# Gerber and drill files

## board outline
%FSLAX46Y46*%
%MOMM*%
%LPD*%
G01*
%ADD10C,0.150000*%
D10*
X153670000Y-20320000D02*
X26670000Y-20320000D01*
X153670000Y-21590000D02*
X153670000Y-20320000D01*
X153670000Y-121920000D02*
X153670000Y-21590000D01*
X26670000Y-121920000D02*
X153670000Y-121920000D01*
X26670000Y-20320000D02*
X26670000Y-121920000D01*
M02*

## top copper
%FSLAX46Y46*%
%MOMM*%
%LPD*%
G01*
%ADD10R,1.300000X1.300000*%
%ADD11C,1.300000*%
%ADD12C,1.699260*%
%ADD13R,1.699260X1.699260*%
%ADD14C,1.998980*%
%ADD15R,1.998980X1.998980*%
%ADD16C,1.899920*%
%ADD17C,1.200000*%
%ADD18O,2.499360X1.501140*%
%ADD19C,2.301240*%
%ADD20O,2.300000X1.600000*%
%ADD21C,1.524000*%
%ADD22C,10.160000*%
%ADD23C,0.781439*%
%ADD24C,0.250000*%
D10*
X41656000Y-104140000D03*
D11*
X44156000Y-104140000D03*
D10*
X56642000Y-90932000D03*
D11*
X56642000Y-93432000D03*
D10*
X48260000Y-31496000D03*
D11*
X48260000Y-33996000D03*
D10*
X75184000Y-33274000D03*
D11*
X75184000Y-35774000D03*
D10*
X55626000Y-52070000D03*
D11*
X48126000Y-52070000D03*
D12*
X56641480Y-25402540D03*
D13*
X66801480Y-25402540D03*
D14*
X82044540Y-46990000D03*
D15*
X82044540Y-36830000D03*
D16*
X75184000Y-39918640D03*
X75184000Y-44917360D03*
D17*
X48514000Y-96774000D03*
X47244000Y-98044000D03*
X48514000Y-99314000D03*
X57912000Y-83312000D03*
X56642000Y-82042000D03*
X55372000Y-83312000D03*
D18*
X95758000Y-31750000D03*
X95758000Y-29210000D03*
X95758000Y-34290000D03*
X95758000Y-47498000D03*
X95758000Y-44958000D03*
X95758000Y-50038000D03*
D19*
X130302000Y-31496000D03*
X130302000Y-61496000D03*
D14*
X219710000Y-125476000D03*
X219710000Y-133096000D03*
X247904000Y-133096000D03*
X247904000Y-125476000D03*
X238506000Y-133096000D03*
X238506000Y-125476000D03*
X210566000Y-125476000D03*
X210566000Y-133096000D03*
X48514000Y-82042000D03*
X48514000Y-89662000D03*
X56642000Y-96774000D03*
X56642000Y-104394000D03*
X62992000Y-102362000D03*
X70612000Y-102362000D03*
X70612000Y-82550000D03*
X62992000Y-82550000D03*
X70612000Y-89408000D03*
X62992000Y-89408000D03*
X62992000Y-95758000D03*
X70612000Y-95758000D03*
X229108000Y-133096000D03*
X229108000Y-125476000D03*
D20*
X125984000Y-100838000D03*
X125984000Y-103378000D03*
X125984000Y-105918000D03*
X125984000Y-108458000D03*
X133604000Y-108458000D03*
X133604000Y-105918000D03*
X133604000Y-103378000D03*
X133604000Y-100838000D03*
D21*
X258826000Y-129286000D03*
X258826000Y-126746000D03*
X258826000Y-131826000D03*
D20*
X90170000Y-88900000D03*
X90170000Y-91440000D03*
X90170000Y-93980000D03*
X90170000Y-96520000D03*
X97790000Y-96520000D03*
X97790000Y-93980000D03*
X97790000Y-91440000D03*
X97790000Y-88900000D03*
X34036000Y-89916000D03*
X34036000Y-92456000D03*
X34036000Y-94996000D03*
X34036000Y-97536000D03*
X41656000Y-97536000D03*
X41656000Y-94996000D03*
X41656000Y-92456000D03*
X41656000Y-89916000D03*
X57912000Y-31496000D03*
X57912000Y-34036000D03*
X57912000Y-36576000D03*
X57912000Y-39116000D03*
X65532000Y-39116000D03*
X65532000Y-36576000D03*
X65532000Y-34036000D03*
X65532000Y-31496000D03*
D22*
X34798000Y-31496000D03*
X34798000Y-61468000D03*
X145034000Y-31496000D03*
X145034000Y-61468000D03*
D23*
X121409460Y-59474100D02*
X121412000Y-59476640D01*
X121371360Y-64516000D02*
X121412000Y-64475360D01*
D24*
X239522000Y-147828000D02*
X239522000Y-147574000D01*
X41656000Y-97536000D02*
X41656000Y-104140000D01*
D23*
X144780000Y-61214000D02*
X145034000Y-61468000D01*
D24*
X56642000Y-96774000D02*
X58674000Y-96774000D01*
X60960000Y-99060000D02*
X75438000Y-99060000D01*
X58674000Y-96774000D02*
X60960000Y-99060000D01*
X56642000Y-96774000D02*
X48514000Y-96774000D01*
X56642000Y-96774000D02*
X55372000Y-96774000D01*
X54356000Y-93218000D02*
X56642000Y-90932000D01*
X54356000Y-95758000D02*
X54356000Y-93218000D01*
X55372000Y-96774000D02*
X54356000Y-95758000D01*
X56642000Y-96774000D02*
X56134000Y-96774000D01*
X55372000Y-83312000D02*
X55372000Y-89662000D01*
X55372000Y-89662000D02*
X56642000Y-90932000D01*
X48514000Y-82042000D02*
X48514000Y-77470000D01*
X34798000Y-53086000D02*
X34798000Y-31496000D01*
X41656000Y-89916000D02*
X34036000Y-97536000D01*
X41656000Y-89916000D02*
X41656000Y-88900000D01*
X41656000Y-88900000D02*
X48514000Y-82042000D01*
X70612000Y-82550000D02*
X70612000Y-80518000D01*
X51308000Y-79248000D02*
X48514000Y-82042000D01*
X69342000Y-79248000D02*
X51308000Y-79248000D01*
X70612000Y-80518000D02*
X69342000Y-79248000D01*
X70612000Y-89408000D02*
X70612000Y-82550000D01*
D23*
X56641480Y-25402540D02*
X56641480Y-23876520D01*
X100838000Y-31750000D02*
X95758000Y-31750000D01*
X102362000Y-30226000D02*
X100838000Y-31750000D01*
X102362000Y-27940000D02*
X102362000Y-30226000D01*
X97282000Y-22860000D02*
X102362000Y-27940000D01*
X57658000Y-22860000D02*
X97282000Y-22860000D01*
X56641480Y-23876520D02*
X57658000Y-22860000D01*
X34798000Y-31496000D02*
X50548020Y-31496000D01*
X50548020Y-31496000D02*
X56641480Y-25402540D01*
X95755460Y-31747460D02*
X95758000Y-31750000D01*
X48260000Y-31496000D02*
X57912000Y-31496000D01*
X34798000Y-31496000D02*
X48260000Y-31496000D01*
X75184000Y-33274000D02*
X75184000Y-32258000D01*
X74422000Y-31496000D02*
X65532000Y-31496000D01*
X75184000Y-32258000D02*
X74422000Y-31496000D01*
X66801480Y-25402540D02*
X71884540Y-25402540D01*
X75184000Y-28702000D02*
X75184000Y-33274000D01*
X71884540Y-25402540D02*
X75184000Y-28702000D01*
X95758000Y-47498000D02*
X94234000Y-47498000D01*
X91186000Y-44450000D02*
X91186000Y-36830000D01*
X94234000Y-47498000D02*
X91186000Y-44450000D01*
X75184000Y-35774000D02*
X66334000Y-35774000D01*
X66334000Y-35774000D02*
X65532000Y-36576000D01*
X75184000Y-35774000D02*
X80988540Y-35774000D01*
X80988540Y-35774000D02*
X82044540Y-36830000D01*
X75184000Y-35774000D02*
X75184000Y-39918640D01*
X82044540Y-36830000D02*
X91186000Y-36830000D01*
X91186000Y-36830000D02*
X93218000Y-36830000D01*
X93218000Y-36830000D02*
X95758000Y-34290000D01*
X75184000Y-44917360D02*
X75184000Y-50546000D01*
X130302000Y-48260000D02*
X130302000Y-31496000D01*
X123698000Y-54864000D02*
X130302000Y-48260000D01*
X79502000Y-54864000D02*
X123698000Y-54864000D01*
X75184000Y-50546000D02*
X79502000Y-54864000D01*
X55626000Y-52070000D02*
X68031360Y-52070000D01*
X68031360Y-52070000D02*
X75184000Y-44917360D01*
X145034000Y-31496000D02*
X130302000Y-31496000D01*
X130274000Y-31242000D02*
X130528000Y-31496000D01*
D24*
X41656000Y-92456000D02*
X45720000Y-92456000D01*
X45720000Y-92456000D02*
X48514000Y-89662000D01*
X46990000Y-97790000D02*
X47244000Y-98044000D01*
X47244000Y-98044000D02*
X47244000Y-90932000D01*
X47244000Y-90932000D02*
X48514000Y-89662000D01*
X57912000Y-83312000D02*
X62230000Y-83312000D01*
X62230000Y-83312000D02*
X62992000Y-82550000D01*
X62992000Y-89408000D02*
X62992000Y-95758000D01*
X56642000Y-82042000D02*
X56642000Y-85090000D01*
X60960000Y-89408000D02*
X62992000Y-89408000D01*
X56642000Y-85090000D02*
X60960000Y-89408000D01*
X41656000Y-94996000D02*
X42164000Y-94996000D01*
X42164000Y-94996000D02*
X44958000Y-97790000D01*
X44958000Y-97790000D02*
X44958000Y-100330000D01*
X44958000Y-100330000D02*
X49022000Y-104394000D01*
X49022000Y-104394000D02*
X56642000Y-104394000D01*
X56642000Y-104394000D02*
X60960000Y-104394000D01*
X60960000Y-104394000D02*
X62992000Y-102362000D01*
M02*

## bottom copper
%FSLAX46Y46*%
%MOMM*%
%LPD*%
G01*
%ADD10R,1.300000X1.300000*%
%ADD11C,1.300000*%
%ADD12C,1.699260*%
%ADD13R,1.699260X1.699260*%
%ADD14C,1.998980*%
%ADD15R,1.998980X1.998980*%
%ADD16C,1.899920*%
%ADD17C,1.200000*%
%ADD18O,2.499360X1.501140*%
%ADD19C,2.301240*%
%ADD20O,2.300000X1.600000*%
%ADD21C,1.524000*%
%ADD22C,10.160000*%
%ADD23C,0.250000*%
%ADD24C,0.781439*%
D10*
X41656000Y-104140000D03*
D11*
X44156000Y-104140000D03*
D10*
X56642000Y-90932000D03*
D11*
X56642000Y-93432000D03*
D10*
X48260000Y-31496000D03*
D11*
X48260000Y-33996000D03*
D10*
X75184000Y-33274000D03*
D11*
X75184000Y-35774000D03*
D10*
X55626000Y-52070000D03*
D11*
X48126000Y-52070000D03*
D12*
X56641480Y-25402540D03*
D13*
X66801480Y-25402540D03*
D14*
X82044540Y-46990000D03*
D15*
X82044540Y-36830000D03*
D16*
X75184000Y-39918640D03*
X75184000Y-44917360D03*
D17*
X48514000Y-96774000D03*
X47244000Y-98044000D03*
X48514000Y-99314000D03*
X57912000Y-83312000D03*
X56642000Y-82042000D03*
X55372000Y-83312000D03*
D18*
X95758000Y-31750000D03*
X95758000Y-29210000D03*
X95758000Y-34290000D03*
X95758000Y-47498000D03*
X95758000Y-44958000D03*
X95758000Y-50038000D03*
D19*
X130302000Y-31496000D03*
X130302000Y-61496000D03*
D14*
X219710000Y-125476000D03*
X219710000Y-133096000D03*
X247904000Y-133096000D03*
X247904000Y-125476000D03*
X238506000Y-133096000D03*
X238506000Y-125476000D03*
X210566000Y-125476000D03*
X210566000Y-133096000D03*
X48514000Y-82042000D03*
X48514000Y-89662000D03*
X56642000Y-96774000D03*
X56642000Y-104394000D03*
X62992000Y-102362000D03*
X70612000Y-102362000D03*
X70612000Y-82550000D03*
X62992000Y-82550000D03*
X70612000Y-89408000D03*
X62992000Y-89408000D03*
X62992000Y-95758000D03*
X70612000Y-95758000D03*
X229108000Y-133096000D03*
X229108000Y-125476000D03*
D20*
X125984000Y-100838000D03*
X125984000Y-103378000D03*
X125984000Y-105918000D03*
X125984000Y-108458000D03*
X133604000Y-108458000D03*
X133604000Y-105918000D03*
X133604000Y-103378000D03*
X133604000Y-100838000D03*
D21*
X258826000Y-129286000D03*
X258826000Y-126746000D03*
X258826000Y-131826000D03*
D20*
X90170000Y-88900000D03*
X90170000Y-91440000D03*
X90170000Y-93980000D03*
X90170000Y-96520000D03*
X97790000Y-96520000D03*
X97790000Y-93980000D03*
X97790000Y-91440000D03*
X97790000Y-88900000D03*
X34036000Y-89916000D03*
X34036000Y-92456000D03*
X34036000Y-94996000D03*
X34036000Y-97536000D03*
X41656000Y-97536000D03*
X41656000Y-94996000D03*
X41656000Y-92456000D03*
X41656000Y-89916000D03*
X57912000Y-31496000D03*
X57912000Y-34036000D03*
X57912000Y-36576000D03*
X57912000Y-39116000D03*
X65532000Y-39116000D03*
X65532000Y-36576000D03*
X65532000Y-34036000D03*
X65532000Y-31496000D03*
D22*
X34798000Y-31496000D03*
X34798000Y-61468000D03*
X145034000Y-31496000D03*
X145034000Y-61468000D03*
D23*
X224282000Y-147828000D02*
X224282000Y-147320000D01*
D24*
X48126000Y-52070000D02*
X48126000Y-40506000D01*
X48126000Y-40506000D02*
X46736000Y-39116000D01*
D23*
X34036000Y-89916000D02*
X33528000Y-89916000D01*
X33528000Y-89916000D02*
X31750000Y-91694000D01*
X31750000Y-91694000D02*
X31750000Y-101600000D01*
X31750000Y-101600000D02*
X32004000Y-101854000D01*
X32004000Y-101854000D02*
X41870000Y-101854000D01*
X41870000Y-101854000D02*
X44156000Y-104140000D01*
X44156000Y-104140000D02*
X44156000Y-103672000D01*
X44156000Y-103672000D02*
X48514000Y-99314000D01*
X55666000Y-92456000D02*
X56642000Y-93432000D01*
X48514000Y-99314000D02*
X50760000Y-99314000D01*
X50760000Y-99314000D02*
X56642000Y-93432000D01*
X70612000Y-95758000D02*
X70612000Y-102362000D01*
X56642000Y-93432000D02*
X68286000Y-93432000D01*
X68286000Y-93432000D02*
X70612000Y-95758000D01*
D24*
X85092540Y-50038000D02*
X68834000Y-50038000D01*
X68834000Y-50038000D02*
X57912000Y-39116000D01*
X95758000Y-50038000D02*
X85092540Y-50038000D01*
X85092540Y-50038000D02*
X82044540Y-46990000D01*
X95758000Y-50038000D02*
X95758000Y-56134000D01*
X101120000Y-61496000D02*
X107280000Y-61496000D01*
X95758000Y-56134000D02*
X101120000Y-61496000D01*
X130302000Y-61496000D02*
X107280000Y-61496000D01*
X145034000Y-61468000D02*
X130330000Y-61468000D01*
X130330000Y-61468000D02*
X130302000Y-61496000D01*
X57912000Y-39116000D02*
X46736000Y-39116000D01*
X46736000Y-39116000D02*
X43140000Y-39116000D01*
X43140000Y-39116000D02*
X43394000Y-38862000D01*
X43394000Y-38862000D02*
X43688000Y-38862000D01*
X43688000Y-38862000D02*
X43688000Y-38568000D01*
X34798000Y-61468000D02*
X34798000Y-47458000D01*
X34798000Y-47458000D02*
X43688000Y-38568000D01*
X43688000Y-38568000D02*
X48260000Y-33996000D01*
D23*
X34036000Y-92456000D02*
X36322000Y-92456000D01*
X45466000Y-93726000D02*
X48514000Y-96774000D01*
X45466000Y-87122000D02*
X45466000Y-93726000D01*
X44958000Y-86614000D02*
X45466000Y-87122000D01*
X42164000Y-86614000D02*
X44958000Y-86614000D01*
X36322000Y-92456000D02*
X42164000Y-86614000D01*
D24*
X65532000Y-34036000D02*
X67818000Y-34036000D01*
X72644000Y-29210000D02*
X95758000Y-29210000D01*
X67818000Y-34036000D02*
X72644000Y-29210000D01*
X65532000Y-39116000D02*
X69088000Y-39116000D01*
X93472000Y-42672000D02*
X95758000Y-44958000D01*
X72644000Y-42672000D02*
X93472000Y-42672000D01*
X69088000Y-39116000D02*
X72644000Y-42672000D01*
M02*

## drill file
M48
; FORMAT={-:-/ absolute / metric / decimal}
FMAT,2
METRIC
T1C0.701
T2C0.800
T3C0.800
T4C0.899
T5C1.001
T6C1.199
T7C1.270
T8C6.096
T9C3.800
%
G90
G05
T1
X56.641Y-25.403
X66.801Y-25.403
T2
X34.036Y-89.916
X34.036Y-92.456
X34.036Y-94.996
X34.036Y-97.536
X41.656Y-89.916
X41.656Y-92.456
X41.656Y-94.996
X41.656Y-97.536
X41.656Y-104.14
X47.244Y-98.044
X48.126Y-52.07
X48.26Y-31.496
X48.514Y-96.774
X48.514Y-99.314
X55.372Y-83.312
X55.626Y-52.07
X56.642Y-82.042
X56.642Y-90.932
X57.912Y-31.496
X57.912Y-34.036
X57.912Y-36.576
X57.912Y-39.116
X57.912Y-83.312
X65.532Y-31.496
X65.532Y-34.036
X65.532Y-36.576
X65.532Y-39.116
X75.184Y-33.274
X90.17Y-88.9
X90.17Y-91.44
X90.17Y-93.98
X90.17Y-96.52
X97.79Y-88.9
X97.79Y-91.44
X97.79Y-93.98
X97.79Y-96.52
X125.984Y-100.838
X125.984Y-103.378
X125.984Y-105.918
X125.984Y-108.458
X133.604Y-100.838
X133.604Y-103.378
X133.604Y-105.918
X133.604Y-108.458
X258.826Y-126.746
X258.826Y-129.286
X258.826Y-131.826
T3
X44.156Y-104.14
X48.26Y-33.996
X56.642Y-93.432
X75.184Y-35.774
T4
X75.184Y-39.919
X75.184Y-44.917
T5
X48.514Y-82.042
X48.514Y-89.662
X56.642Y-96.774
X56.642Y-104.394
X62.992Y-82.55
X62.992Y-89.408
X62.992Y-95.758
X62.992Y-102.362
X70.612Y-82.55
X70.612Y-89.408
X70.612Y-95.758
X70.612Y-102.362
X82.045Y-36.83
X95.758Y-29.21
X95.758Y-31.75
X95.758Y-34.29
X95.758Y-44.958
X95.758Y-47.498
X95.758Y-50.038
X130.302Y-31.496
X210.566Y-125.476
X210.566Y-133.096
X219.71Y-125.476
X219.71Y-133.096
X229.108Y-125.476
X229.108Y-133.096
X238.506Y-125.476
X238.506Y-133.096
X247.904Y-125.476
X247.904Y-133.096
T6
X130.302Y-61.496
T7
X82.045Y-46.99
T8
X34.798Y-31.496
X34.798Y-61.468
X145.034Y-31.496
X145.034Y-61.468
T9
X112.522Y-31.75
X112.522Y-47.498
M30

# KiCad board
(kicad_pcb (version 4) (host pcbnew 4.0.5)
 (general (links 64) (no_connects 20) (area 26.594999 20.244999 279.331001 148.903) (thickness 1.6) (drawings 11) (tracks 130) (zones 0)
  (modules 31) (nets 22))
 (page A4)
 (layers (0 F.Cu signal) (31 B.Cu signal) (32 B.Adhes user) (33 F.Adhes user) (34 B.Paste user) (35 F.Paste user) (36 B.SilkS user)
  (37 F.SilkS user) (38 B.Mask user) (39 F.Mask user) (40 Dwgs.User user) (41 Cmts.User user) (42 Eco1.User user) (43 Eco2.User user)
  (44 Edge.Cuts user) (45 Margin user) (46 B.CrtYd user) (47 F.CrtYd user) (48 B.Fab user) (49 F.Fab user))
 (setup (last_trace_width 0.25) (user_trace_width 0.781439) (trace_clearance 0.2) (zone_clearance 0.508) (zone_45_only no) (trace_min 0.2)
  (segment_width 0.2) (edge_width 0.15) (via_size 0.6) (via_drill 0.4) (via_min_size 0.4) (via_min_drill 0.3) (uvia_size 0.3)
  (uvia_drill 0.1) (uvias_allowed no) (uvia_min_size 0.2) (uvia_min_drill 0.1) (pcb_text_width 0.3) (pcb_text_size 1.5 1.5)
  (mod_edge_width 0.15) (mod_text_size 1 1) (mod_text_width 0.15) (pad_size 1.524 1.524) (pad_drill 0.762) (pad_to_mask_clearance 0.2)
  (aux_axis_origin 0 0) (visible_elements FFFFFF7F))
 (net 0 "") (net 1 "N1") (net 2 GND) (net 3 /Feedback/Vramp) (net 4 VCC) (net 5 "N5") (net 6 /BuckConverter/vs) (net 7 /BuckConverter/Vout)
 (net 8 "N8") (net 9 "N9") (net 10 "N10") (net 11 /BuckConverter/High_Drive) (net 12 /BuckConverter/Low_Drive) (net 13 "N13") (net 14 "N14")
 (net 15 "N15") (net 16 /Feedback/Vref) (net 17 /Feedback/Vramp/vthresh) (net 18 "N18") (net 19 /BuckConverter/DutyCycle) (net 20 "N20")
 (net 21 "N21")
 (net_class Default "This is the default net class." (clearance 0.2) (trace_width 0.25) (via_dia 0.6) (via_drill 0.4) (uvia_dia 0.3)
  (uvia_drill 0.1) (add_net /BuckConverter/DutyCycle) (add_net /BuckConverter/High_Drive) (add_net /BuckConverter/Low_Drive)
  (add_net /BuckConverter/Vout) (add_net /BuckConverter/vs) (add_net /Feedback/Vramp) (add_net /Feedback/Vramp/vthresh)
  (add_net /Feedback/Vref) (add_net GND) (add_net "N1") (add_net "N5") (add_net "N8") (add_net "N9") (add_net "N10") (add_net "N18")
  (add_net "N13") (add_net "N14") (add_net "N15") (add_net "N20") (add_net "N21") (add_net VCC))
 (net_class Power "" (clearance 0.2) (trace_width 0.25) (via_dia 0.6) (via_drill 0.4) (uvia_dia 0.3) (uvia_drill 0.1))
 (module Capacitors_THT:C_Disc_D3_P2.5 (layer F.Cu) (at 41.656 104.14)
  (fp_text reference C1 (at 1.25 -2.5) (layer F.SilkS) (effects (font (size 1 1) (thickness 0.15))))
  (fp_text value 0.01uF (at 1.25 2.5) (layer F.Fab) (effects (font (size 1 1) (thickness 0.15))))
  (pad 1 thru_hole rect (at 0 0) (size 1.3 1.3) (drill 0.8) (layers *.Cu *.Mask) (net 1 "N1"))
  (pad 2 thru_hole circle (at 2.5 0) (size 1.3 1.3) (drill 0.8001) (layers *.Cu *.Mask) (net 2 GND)))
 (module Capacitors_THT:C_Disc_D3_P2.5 (layer F.Cu) (at 56.642 90.932 270)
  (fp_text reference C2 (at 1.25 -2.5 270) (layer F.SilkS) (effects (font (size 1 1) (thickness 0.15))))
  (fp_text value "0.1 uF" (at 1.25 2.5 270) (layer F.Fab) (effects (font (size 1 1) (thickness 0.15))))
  (pad 1 thru_hole rect (at 0 0 270) (size 1.3 1.3) (drill 0.8) (layers *.Cu *.Mask) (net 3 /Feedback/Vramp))
  (pad 2 thru_hole circle (at 2.5 0 270) (size 1.3 1.3) (drill 0.8001) (layers *.Cu *.Mask) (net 2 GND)))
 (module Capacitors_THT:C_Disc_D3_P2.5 (layer F.Cu) (at 48.26 31.496 270)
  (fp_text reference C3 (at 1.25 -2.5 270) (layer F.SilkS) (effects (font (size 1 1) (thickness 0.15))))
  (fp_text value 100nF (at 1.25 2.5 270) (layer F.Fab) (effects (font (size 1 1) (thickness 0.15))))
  (pad 1 thru_hole rect (at 0 0 270) (size 1.3 1.3) (drill 0.8) (layers *.Cu *.Mask) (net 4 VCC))
  (pad 2 thru_hole circle (at 2.5 0 270) (size 1.3 1.3) (drill 0.8001) (layers *.Cu *.Mask) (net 2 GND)))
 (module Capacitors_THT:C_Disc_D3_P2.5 (layer F.Cu) (at 75.184 33.274 270)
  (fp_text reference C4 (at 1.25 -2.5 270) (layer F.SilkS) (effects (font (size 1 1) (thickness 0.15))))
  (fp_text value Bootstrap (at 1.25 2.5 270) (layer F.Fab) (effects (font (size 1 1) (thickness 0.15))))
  (pad 1 thru_hole rect (at 0 0 270) (size 1.3 1.3) (drill 0.8) (layers *.Cu *.Mask) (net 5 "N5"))
  (pad 2 thru_hole circle (at 2.5 0 270) (size 1.3 1.3) (drill 0.8001) (layers *.Cu *.Mask) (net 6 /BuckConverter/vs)))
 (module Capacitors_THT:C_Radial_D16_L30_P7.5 (layer F.Cu) (at 55.626 52.07 180)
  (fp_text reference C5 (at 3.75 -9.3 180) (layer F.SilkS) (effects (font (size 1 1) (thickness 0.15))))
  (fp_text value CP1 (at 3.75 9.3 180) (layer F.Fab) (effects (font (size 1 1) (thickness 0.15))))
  (pad 1 thru_hole rect (at 0 0 180) (size 1.3 1.3) (drill 0.8) (layers *.Cu *.Mask) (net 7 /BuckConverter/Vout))
  (pad 2 thru_hole circle (at 7.5 0 180) (size 1.3 1.3) (drill 0.8) (layers *.Cu *.Mask) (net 2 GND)))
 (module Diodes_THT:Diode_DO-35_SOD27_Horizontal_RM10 (layer F.Cu) (at 66.802 25.4 180)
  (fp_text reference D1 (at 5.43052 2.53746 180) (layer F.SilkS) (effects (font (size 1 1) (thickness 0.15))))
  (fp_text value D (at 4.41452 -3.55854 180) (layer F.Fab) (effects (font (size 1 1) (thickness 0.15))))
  (pad 2 thru_hole circle (at 10.16052 -0.00254) (size 1.69926 1.69926) (drill 0.70104) (layers *.Cu *.Mask) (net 4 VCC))
  (pad 1 thru_hole rect (at 0.00052 -0.00254) (size 1.69926 1.69926) (drill 0.70104) (layers *.Cu *.Mask) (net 5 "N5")))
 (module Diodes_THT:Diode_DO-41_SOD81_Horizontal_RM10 (layer F.Cu) (at 82.042 36.83 270)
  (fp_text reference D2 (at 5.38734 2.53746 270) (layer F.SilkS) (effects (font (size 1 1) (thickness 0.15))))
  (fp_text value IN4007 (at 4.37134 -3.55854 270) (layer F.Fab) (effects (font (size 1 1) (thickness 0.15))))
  (pad 2 thru_hole circle (at 10.16 -0.00254 90) (size 1.99898 1.99898) (drill 1.27) (layers *.Cu *.Mask) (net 2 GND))
  (pad 1 thru_hole rect (at 0 -0.00254 90) (size 1.99898 1.99898) (drill 1.00076) (layers *.Cu *.Mask) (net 6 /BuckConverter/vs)))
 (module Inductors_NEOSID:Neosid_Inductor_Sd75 (layer F.Cu) (at 75.184 42.418 90)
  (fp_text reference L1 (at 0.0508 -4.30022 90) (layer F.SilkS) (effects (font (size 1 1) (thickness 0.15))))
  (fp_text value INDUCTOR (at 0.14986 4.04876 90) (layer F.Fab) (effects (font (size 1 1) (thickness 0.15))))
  (pad 2 thru_hole circle (at 2.49936 0 90) (size 1.89992 1.89992) (drill 0.89916) (layers *.Cu *.Mask) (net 6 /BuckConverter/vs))
  (pad 1 thru_hole circle (at -2.49936 0 90) (size 1.89992 1.89992) (drill 0.89916) (layers *.Cu *.Mask) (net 7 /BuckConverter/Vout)))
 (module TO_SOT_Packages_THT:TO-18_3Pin (layer F.Cu) (at 48.514 98.044 90)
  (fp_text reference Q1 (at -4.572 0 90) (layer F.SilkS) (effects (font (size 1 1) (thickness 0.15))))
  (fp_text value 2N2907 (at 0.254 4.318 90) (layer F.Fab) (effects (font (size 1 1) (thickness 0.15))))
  (pad 1 thru_hole circle (at 1.27 0 90) (size 1.2 1.2) (drill 0.8) (layers *.Cu *.Mask) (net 3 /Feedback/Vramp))
  (pad 2 thru_hole circle (at 0 -1.27 90) (size 1.2 1.2) (drill 0.8) (layers *.Cu *.Mask) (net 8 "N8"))
  (pad 3 thru_hole circle (at -1.27 0 90) (size 1.2 1.2) (drill 0.8) (layers *.Cu *.Mask) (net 2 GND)))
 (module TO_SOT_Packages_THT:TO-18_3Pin (layer F.Cu) (at 56.642 83.312)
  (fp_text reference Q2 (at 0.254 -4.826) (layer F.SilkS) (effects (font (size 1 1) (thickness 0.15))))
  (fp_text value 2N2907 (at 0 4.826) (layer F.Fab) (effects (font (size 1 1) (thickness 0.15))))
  (pad 1 thru_hole circle (at 1.27 0) (size 1.2 1.2) (drill 0.8) (layers *.Cu *.Mask) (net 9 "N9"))
  (pad 2 thru_hole circle (at 0 -1.27) (size 1.2 1.2) (drill 0.8) (layers *.Cu *.Mask) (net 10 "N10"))
  (pad 3 thru_hole circle (at -1.27 0) (size 1.2 1.2) (drill 0.8) (layers *.Cu *.Mask) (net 3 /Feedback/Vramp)))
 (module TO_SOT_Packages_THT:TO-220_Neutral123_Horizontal (layer F.Cu) (at 95.758 31.75 270)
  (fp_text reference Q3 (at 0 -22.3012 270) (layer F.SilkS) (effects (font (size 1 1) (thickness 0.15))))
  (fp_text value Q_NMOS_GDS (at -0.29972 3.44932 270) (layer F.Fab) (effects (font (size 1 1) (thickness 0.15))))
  (pad 2 thru_hole oval (at 0 0) (size 2.49936 1.50114) (drill 1.00076) (layers *.Cu *.Mask) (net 4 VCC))
  (pad 1 thru_hole oval (at -2.54 0) (size 2.49936 1.50114) (drill 1.00076) (layers *.Cu *.Mask) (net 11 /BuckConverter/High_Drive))
  (pad 3 thru_hole oval (at 2.54 0) (size 2.49936 1.50114) (drill 1.00076) (layers *.Cu *.Mask) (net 6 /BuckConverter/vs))
  (pad "" np_thru_hole circle (at 0 -16.764) (size 3.79984 3.79984) (drill 3.79984) (layers *.Cu *.Mask)))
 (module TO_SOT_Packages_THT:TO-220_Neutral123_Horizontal (layer F.Cu) (at 95.758 47.498 270)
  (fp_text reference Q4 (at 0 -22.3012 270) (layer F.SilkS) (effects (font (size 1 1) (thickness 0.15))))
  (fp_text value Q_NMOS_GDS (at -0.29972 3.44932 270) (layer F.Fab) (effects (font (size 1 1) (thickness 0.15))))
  (pad 2 thru_hole oval (at 0 0) (size 2.49936 1.50114) (drill 1.00076) (layers *.Cu *.Mask) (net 6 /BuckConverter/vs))
  (pad 1 thru_hole oval (at -2.54 0) (size 2.49936 1.50114) (drill 1.00076) (layers *.Cu *.Mask) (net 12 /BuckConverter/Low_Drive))
  (pad 3 thru_hole oval (at 2.54 0) (size 2.49936 1.50114) (drill 1.00076) (layers *.Cu *.Mask) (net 2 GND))
  (pad "" np_thru_hole circle (at 0 -16.764) (size 3.79984 3.79984) (drill 3.79984) (layers *.Cu *.Mask)))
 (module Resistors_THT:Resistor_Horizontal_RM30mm (layer F.Cu) (at 130.302 31.496 270)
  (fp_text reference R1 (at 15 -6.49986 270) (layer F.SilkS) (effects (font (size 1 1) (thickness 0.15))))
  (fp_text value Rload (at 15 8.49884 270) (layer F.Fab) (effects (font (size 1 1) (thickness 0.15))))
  (pad 1 thru_hole circle (at 0 0 270) (size 2.30124 2.30124) (drill 1.00076) (layers *.Cu *.SilkS *.Mask) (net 7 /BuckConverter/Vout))
  (pad 2 thru_hole circle (at 30 0 270) (size 2.30124 2.30124) (drill 1.19888) (layers *.Cu *.SilkS *.Mask) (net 2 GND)))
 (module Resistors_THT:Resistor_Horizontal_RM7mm (layer F.Cu) (at 219.71 125.476 270)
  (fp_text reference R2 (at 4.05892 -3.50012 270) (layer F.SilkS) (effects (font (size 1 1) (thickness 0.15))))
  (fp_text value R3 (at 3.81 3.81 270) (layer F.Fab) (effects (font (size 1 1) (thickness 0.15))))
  (pad 1 thru_hole circle (at 0 0 270) (size 1.99898 1.99898) (drill 1.00076) (layers *.Cu *.SilkS *.Mask) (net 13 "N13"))
  (pad 2 thru_hole circle (at 7.62 0 270) (size 1.99898 1.99898) (drill 1.00076) (layers *.Cu *.SilkS *.Mask) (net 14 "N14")))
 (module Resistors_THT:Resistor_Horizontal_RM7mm (layer F.Cu) (at 247.904 133.096 90)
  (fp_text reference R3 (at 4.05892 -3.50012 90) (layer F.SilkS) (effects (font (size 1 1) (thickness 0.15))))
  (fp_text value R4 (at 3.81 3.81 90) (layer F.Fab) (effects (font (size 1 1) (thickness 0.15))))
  (pad 1 thru_hole circle (at 0 0 90) (size 1.99898 1.99898) (drill 1.00076) (layers *.Cu *.SilkS *.Mask) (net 2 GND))
  (pad 2 thru_hole circle (at 7.62 0 90) (size 1.99898 1.99898) (drill 1.00076) (layers *.Cu *.SilkS *.Mask) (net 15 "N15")))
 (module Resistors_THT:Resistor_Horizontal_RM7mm (layer F.Cu) (at 238.506 133.096 90)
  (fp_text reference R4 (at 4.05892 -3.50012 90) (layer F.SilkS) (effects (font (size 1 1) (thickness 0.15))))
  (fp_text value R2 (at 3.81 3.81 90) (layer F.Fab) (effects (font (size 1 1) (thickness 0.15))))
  (pad 1 thru_hole circle (at 0 0 90) (size 1.99898 1.99898) (drill 1.00076) (layers *.Cu *.SilkS *.Mask) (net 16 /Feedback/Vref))
  (pad 2 thru_hole circle (at 7.62 0 90) (size 1.99898 1.99898) (drill 1.00076) (layers *.Cu *.SilkS *.Mask) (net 15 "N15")))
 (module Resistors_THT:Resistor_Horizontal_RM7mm (layer F.Cu) (at 210.566 125.476 270)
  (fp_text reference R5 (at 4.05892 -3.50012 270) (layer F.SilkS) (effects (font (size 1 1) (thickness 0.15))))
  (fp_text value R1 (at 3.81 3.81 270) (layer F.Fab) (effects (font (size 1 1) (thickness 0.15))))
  (pad 1 thru_hole circle (at 0 0 270) (size 1.99898 1.99898) (drill 1.00076) (layers *.Cu *.SilkS *.Mask) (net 7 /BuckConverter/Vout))
  (pad 2 thru_hole circle (at 7.62 0 270) (size 1.99898 1.99898) (drill 1.00076) (layers *.Cu *.SilkS *.Mask) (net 13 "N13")))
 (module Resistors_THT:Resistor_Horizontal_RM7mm (layer F.Cu) (at 48.514 82.042 270)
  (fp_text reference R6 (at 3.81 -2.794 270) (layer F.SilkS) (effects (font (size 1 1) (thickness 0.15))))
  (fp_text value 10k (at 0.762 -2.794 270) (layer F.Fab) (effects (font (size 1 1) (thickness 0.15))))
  (pad 1 thru_hole circle (at 0 0 270) (size 1.99898 1.99898) (drill 1.00076) (layers *.Cu *.SilkS *.Mask) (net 4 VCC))
  (pad 2 thru_hole circle (at 7.62 0 270) (size 1.99898 1.99898) (drill 1.00076) (layers *.Cu *.SilkS *.Mask) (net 8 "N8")))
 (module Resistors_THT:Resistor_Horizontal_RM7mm (layer F.Cu) (at 56.642 96.774 270)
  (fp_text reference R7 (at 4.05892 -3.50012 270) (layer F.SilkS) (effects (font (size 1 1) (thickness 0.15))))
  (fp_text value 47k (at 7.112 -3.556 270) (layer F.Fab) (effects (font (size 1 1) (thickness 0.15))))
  (pad 1 thru_hole circle (at 0 0 270) (size 1.99898 1.99898) (drill 1.00076) (layers *.Cu *.SilkS *.Mask) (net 3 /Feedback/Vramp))
  (pad 2 thru_hole circle (at 7.62 0 270) (size 1.99898 1.99898) (drill 1.00076) (layers *.Cu *.SilkS *.Mask)
   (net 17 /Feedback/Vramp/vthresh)))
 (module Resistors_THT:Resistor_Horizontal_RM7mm (layer F.Cu) (at 62.992 102.362)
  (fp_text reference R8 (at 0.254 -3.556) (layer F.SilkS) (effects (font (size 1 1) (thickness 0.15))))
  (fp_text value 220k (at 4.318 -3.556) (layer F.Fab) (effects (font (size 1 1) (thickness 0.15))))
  (pad 1 thru_hole circle (at 0 0) (size 1.99898 1.99898) (drill 1.00076) (layers *.Cu *.SilkS *.Mask) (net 17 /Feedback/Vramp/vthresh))
  (pad 2 thru_hole circle (at 7.62 0) (size 1.99898 1.99898) (drill 1.00076) (layers *.Cu *.SilkS *.Mask) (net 2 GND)))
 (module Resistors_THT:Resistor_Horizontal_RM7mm (layer F.Cu) (at 70.612 82.55 180)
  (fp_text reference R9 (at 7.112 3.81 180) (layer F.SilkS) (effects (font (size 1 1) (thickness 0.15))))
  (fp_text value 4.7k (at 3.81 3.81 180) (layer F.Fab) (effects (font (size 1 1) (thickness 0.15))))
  (pad 1 thru_hole circle (at 0 0 180) (size 1.99898 1.99898) (drill 1.00076) (layers *.Cu *.SilkS *.Mask) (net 4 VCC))
  (pad 2 thru_hole circle (at 7.62 0 180) (size 1.99898 1.99898) (drill 1.00076) (layers *.Cu *.SilkS *.Mask) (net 9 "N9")))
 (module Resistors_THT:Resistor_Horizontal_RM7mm (layer F.Cu) (at 70.612 89.408 180)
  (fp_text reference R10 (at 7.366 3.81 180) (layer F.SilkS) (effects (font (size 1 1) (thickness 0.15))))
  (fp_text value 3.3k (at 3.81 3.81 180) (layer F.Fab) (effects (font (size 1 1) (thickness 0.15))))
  (pad 1 thru_hole circle (at 0 0 180) (size 1.99898 1.99898) (drill 1.00076) (layers *.Cu *.SilkS *.Mask) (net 4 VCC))
  (pad 2 thru_hole circle (at 7.62 0 180) (size 1.99898 1.99898) (drill 1.00076) (layers *.Cu *.SilkS *.Mask) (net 10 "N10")))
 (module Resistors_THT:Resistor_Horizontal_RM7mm (layer F.Cu) (at 62.992 95.758)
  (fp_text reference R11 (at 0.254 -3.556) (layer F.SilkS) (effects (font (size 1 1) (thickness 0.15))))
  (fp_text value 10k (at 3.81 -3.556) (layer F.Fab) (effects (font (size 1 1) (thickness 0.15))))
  (pad 1 thru_hole circle (at 0 0) (size 1.99898 1.99898) (drill 1.00076) (layers *.Cu *.SilkS *.Mask) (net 10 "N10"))
  (pad 2 thru_hole circle (at 7.62 0) (size 1.99898 1.99898) (drill 1.00076) (layers *.Cu *.SilkS *.Mask) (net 2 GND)))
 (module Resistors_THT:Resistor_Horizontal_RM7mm (layer F.Cu) (at 229.108 133.096 90)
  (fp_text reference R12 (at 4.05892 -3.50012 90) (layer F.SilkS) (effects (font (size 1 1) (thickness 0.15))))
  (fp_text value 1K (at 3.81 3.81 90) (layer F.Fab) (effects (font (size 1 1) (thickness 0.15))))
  (pad 1 thru_hole circle (at 0 0 90) (size 1.99898 1.99898) (drill 1.00076) (layers *.Cu *.SilkS *.Mask) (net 4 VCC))
  (pad 2 thru_hole circle (at 7.62 0 90) (size 1.99898 1.99898) (drill 1.00076) (layers *.Cu *.SilkS *.Mask) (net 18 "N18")))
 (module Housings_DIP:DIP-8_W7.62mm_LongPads (layer F.Cu) (at 125.984 100.838)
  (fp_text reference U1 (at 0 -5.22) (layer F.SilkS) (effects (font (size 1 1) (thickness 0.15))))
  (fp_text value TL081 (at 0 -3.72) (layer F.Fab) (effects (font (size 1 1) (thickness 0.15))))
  (pad 1 thru_hole oval (at 0 0) (size 2.3 1.6) (drill 0.8) (layers *.Cu *.Mask))
  (pad 2 thru_hole oval (at 0 2.54) (size 2.3 1.6) (drill 0.8) (layers *.Cu *.Mask) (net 3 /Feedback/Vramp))
  (pad 3 thru_hole oval (at 0 5.08) (size 2.3 1.6) (drill 0.8) (layers *.Cu *.Mask) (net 14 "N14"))
  (pad 4 thru_hole oval (at 0 7.62) (size 2.3 1.6) (drill 0.8) (layers *.Cu *.Mask) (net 2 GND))
  (pad 5 thru_hole oval (at 7.62 7.62) (size 2.3 1.6) (drill 0.8) (layers *.Cu *.Mask))
  (pad 6 thru_hole oval (at 7.62 5.08) (size 2.3 1.6) (drill 0.8) (layers *.Cu *.Mask) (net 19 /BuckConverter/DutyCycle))
  (pad 7 thru_hole oval (at 7.62 2.54) (size 2.3 1.6) (drill 0.8) (layers *.Cu *.Mask) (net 4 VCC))
  (pad 8 thru_hole oval (at 7.62 0) (size 2.3 1.6) (drill 0.8) (layers *.Cu *.Mask)))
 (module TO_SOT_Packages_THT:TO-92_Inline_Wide (layer F.Cu) (at 258.826 131.826 90)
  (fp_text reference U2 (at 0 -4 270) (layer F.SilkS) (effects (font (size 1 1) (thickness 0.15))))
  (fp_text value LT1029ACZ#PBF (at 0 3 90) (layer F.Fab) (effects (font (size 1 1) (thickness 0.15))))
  (pad 2 thru_hole circle (at 2.54 0 180) (size 1.524 1.524) (drill 0.8) (layers *.Cu *.Mask) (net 16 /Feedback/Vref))
  (pad 3 thru_hole circle (at 5.08 0 180) (size 1.524 1.524) (drill 0.8) (layers *.Cu *.Mask) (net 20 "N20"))
  (pad 1 thru_hole circle (at 0 0 180) (size 1.524 1.524) (drill 0.8) (layers *.Cu *.Mask) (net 2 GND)))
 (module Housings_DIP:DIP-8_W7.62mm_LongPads (layer F.Cu) (at 90.17 88.9)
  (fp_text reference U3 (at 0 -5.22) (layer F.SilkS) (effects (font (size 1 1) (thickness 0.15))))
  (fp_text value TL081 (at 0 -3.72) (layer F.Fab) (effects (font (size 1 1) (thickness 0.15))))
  (pad 1 thru_hole oval (at 0 0) (size 2.3 1.6) (drill 0.8) (layers *.Cu *.Mask))
  (pad 2 thru_hole oval (at 0 2.54) (size 2.3 1.6) (drill 0.8) (layers *.Cu *.Mask) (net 13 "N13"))
  (pad 3 thru_hole oval (at 0 5.08) (size 2.3 1.6) (drill 0.8) (layers *.Cu *.Mask) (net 15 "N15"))
  (pad 4 thru_hole oval (at 0 7.62) (size 2.3 1.6) (drill 0.8) (layers *.Cu *.Mask) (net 2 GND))
  (pad 5 thru_hole oval (at 7.62 7.62) (size 2.3 1.6) (drill 0.8) (layers *.Cu *.Mask))
  (pad 6 thru_hole oval (at 7.62 5.08) (size 2.3 1.6) (drill 0.8) (layers *.Cu *.Mask) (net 14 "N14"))
  (pad 7 thru_hole oval (at 7.62 2.54) (size 2.3 1.6) (drill 0.8) (layers *.Cu *.Mask) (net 4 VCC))
  (pad 8 thru_hole oval (at 7.62 0) (size 2.3 1.6) (drill 0.8) (layers *.Cu *.Mask)))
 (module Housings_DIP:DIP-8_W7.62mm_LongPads (layer F.Cu) (at 34.036 89.916)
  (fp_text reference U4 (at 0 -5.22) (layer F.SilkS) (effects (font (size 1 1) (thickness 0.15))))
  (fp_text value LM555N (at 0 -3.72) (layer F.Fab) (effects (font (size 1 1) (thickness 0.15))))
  (pad 1 thru_hole oval (at 0 0) (size 2.3 1.6) (drill 0.8) (layers *.Cu *.Mask) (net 2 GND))
  (pad 2 thru_hole oval (at 0 2.54) (size 2.3 1.6) (drill 0.8) (layers *.Cu *.Mask) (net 3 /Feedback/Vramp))
  (pad 3 thru_hole oval (at 0 5.08) (size 2.3 1.6) (drill 0.8) (layers *.Cu *.Mask) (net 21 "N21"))
  (pad 4 thru_hole oval (at 0 7.62) (size 2.3 1.6) (drill 0.8) (layers *.Cu *.Mask) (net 4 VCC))
  (pad 5 thru_hole oval (at 7.62 7.62) (size 2.3 1.6) (drill 0.8) (layers *.Cu *.Mask) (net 1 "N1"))
  (pad 6 thru_hole oval (at 7.62 5.08) (size 2.3 1.6) (drill 0.8) (layers *.Cu *.Mask) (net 17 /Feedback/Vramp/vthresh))
  (pad 7 thru_hole oval (at 7.62 2.54) (size 2.3 1.6) (drill 0.8) (layers *.Cu *.Mask) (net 8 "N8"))
  (pad 8 thru_hole oval (at 7.62 0) (size 2.3 1.6) (drill 0.8) (layers *.Cu *.Mask) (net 4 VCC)))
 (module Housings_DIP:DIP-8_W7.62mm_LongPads (layer F.Cu) (at 57.912 31.496)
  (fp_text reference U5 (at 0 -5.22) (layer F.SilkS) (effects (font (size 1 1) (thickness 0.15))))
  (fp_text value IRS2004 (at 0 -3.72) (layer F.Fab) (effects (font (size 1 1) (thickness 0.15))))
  (pad 1 thru_hole oval (at 0 0) (size 2.3 1.6) (drill 0.8) (layers *.Cu *.Mask) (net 4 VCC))
  (pad 2 thru_hole oval (at 0 2.54) (size 2.3 1.6) (drill 0.8) (layers *.Cu *.Mask) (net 19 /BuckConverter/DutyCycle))
  (pad 3 thru_hole oval (at 0 5.08) (size 2.3 1.6) (drill 0.8) (layers *.Cu *.Mask) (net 18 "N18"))
  (pad 4 thru_hole oval (at 0 7.62) (size 2.3 1.6) (drill 0.8) (layers *.Cu *.Mask) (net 2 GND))
  (pad 5 thru_hole oval (at 7.62 7.62) (size 2.3 1.6) (drill 0.8) (layers *.Cu *.Mask) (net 12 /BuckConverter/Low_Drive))
  (pad 6 thru_hole oval (at 7.62 5.08) (size 2.3 1.6) (drill 0.8) (layers *.Cu *.Mask) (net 6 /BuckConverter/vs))
  (pad 7 thru_hole oval (at 7.62 2.54) (size 2.3 1.6) (drill 0.8) (layers *.Cu *.Mask) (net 11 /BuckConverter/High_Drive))
  (pad 8 thru_hole oval (at 7.62 0) (size 2.3 1.6) (drill 0.8) (layers *.Cu *.Mask) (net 5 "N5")))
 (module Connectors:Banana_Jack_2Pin (layer F.Cu) (at 34.798 46.482 270)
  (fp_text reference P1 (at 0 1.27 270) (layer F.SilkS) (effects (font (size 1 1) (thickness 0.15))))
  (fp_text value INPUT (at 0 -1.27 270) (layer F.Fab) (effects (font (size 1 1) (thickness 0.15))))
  (pad 1 thru_hole circle (at -14.986 0 270) (size 10.16 10.16) (drill 6.096) (layers *.Cu *.Mask) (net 4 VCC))
  (pad 2 thru_hole circle (at 14.986 0 270) (size 10.16 10.16) (drill 6.096) (layers *.Cu *.Mask) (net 2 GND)))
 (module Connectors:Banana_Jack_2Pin (layer F.Cu) (at 145.034 46.482 270)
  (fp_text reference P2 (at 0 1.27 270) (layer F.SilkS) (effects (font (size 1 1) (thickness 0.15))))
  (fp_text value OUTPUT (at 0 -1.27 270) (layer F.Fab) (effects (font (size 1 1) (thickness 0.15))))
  (pad 1 thru_hole circle (at -14.986 0 270) (size 10.16 10.16) (drill 6.096) (layers *.Cu *.Mask) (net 7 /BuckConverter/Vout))
  (pad 2 thru_hole circle (at 14.986 0 270) (size 10.16 10.16) (drill 6.096) (layers *.Cu *.Mask) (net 2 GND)))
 (gr_line (start 153.67 20.32) (end 26.67 20.32) (angle 90) (layer Edge.Cuts) (width 0.15))
 (gr_line (start 153.67 21.59) (end 153.67 20.32) (angle 90) (layer Edge.Cuts) (width 0.15))
 (gr_line (start 153.67 121.92) (end 153.67 21.59) (angle 90) (layer Edge.Cuts) (width 0.15))
 (gr_line (start 26.67 121.92) (end 153.67 121.92) (angle 90) (layer Edge.Cuts) (width 0.15))
 (gr_line (start 26.67 20.32) (end 26.67 121.92) (angle 90) (layer Edge.Cuts) (width 0.15))
 (segment (start 121.40946 59.4741) (end 121.412 59.47664) (width 0.781439) (layer F.Cu) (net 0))
 (segment (start 121.37136 64.516) (end 121.412 64.47536) (width 0.781439) (layer F.Cu) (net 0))
 (segment (start 224.282 147.828) (end 224.282 147.32) (width 0.25) (layer B.Cu) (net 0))
 (segment (start 239.522 147.828) (end 239.522 147.574) (width 0.25) (layer F.Cu) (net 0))
 (segment (start 41.656 97.536) (end 41.656 104.14) (width 0.25) (layer F.Cu) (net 1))
 (segment (start 48.126 52.07) (end 48.126 40.506) (width 0.781439) (layer B.Cu) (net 2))
 (segment (start 48.126 40.506) (end 46.736 39.116) (width 0.781439) (layer B.Cu) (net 2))
 (segment (start 34.036 89.916) (end 33.528 89.916) (width 0.25) (layer B.Cu) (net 2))
 (segment (start 33.528 89.916) (end 31.75 91.694) (width 0.25) (layer B.Cu) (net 2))
 (segment (start 31.75 91.694) (end 31.75 101.6) (width 0.25) (layer B.Cu) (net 2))
 (segment (start 31.75 101.6) (end 32.004 101.854) (width 0.25) (layer B.Cu) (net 2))
 (segment (start 32.004 101.854) (end 41.87 101.854) (width 0.25) (layer B.Cu) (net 2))
 (segment (start 41.87 101.854) (end 44.156 104.14) (width 0.25) (layer B.Cu) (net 2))
 (segment (start 44.156 104.14) (end 44.156 103.672) (width 0.25) (layer B.Cu) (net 2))
 (segment (start 44.156 103.672) (end 48.514 99.314) (width 0.25) (layer B.Cu) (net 2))
 (segment (start 55.666 92.456) (end 56.642 93.432) (width 0.25) (layer B.Cu) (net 2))
 (segment (start 48.514 99.314) (end 50.76 99.314) (width 0.25) (layer B.Cu) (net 2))
 (segment (start 50.76 99.314) (end 56.642 93.432) (width 0.25) (layer B.Cu) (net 2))
 (segment (start 70.612 95.758) (end 70.612 102.362) (width 0.25) (layer B.Cu) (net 2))
 (segment (start 56.642 93.432) (end 68.286 93.432) (width 0.25) (layer B.Cu) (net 2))
 (segment (start 68.286 93.432) (end 70.612 95.758) (width 0.25) (layer B.Cu) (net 2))
 (segment (start 85.09254 50.038) (end 68.834 50.038) (width 0.781439) (layer B.Cu) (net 2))
 (segment (start 68.834 50.038) (end 57.912 39.116) (width 0.781439) (layer B.Cu) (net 2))
 (segment (start 95.758 50.038) (end 85.09254 50.038) (width 0.781439) (layer B.Cu) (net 2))
 (segment (start 85.09254 50.038) (end 82.04454 46.99) (width 0.781439) (layer B.Cu) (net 2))
 (segment (start 95.758 50.038) (end 95.758 56.134) (width 0.781439) (layer B.Cu) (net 2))
 (segment (start 101.12 61.496) (end 107.28 61.496) (width 0.781439) (layer B.Cu) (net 2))
 (segment (start 95.758 56.134) (end 101.12 61.496) (width 0.781439) (layer B.Cu) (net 2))
 (segment (start 130.302 61.496) (end 107.28 61.496) (width 0.781439) (layer B.Cu) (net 2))
 (segment (start 145.034 61.468) (end 130.33 61.468) (width 0.781439) (layer B.Cu) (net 2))
 (segment (start 130.33 61.468) (end 130.302 61.496) (width 0.781439) (layer B.Cu) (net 2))
 (segment (start 57.912 39.116) (end 46.736 39.116) (width 0.781439) (layer B.Cu) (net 2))
 (segment (start 46.736 39.116) (end 43.14 39.116) (width 0.781439) (layer B.Cu) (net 2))
 (segment (start 43.14 39.116) (end 43.394 38.862) (width 0.781439) (layer B.Cu) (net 2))
 (segment (start 43.394 38.862) (end 43.688 38.862) (width 0.781439) (layer B.Cu) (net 2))
 (segment (start 43.688 38.862) (end 43.688 38.568) (width 0.781439) (layer B.Cu) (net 2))
 (segment (start 34.798 61.468) (end 34.798 47.458) (width 0.781439) (layer B.Cu) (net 2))
 (segment (start 34.798 47.458) (end 43.688 38.568) (width 0.781439) (layer B.Cu) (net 2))
 (segment (start 43.688 38.568) (end 48.26 33.996) (width 0.781439) (layer B.Cu) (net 2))
 (segment (start 144.78 61.214) (end 145.034 61.468) (width 0.781439) (layer F.Cu) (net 2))
 (segment (start 56.642 96.774) (end 58.674 96.774) (width 0.25) (layer F.Cu) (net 3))
 (segment (start 60.96 99.06) (end 75.438 99.06) (width 0.25) (layer F.Cu) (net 3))
 (segment (start 58.674 96.774) (end 60.96 99.06) (width 0.25) (layer F.Cu) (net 3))
 (segment (start 34.036 92.456) (end 36.322 92.456) (width 0.25) (layer B.Cu) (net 3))
 (segment (start 45.466 93.726) (end 48.514 96.774) (width 0.25) (layer B.Cu) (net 3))
 (segment (start 45.466 87.122) (end 45.466 93.726) (width 0.25) (layer B.Cu) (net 3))
 (segment (start 44.958 86.614) (end 45.466 87.122) (width 0.25) (layer B.Cu) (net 3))
 (segment (start 42.164 86.614) (end 44.958 86.614) (width 0.25) (layer B.Cu) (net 3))
 (segment (start 36.322 92.456) (end 42.164 86.614) (width 0.25) (layer B.Cu) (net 3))
 (segment (start 56.642 96.774) (end 48.514 96.774) (width 0.25) (layer F.Cu) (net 3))
 (segment (start 56.642 96.774) (end 55.372 96.774) (width 0.25) (layer F.Cu) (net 3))
 (segment (start 54.356 93.218) (end 56.642 90.932) (width 0.25) (layer F.Cu) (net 3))
 (segment (start 54.356 95.758) (end 54.356 93.218) (width 0.25) (layer F.Cu) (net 3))
 (segment (start 55.372 96.774) (end 54.356 95.758) (width 0.25) (layer F.Cu) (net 3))
 (segment (start 56.642 96.774) (end 56.134 96.774) (width 0.25) (layer F.Cu) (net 3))
 (segment (start 55.372 83.312) (end 55.372 89.662) (width 0.25) (layer F.Cu) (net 3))
 (segment (start 55.372 89.662) (end 56.642 90.932) (width 0.25) (layer F.Cu) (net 3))
 (segment (start 48.514 82.042) (end 48.514 77.47) (width 0.25) (layer F.Cu) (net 4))
 (segment (start 34.798 53.086) (end 34.798 31.496) (width 0.25) (layer F.Cu) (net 4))
 (segment (start 41.656 89.916) (end 34.036 97.536) (width 0.25) (layer F.Cu) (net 4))
 (segment (start 41.656 89.916) (end 41.656 88.9) (width 0.25) (layer F.Cu) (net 4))
 (segment (start 41.656 88.9) (end 48.514 82.042) (width 0.25) (layer F.Cu) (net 4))
 (segment (start 70.612 82.55) (end 70.612 80.518) (width 0.25) (layer F.Cu) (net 4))
 (segment (start 51.308 79.248) (end 48.514 82.042) (width 0.25) (layer F.Cu) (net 4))
 (segment (start 69.342 79.248) (end 51.308 79.248) (width 0.25) (layer F.Cu) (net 4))
 (segment (start 70.612 80.518) (end 69.342 79.248) (width 0.25) (layer F.Cu) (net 4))
 (segment (start 70.612 89.408) (end 70.612 82.55) (width 0.25) (layer F.Cu) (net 4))
 (segment (start 56.64148 25.40254) (end 56.64148 23.87652) (width 0.781439) (layer F.Cu) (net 4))
 (segment (start 100.838 31.75) (end 95.758 31.75) (width 0.781439) (layer F.Cu) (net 4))
 (segment (start 102.362 30.226) (end 100.838 31.75) (width 0.781439) (layer F.Cu) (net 4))
 (segment (start 102.362 27.94) (end 102.362 30.226) (width 0.781439) (layer F.Cu) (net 4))
 (segment (start 97.282 22.86) (end 102.362 27.94) (width 0.781439) (layer F.Cu) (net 4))
 (segment (start 57.658 22.86) (end 97.282 22.86) (width 0.781439) (layer F.Cu) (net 4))
 (segment (start 56.64148 23.87652) (end 57.658 22.86) (width 0.781439) (layer F.Cu) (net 4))
 (segment (start 34.798 31.496) (end 50.54802 31.496) (width 0.781439) (layer F.Cu) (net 4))
 (segment (start 50.54802 31.496) (end 56.64148 25.40254) (width 0.781439) (layer F.Cu) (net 4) (status 20))
 (segment (start 95.75546 31.74746) (end 95.758 31.75) (width 0.781439) (layer F.Cu) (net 4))
 (segment (start 48.26 31.496) (end 57.912 31.496) (width 0.781439) (layer F.Cu) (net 4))
 (segment (start 34.798 31.496) (end 48.26 31.496) (width 0.781439) (layer F.Cu) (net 4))
 (segment (start 75.184 33.274) (end 75.184 32.258) (width 0.781439) (layer F.Cu) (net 5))
 (segment (start 74.422 31.496) (end 65.532 31.496) (width 0.781439) (layer F.Cu) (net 5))
 (segment (start 75.184 32.258) (end 74.422 31.496) (width 0.781439) (layer F.Cu) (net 5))
 (segment (start 66.80148 25.40254) (end 71.88454 25.40254) (width 0.781439) (layer F.Cu) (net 5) (status 10))
 (segment (start 75.184 28.702) (end 75.184 33.274) (width 0.781439) (layer F.Cu) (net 5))
 (segment (start 71.88454 25.40254) (end 75.184 28.702) (width 0.781439) (layer F.Cu) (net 5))
 (segment (start 95.758 47.498) (end 94.234 47.498) (width 0.781439) (layer F.Cu) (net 6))
 (segment (start 91.186 44.45) (end 91.186 36.83) (width 0.781439) (layer F.Cu) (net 6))
 (segment (start 94.234 47.498) (end 91.186 44.45) (width 0.781439) (layer F.Cu) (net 6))
 (segment (start 75.184 35.774) (end 66.334 35.774) (width 0.781439) (layer F.Cu) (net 6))
 (segment (start 66.334 35.774) (end 65.532 36.576) (width 0.781439) (layer F.Cu) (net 6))
 (segment (start 75.184 35.774) (end 80.98854 35.774) (width 0.781439) (layer F.Cu) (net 6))
 (segment (start 80.98854 35.774) (end 82.04454 36.83) (width 0.781439) (layer F.Cu) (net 6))
 (segment (start 75.184 35.774) (end 75.184 39.91864) (width 0.781439) (layer F.Cu) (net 6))
 (segment (start 82.04454 36.83) (end 91.186 36.83) (width 0.781439) (layer F.Cu) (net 6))
 (segment (start 91.186 36.83) (end 93.218 36.83) (width 0.781439) (layer F.Cu) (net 6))
 (segment (start 93.218 36.83) (end 95.758 34.29) (width 0.781439) (layer F.Cu) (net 6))
 (segment (start 75.184 44.91736) (end 75.184 50.546) (width 0.781439) (layer F.Cu) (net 7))
 (segment (start 130.302 48.26) (end 130.302 31.496) (width 0.781439) (layer F.Cu) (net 7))
 (segment (start 123.698 54.864) (end 130.302 48.26) (width 0.781439) (layer F.Cu) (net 7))
 (segment (start 79.502 54.864) (end 123.698 54.864) (width 0.781439) (layer F.Cu) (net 7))
 (segment (start 75.184 50.546) (end 79.502 54.864) (width 0.781439) (layer F.Cu) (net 7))
 (segment (start 55.626 52.07) (end 68.03136 52.07) (width 0.781439) (layer F.Cu) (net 7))
 (segment (start 68.03136 52.07) (end 75.184 44.91736) (width 0.781439) (layer F.Cu) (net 7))
 (segment (start 145.034 31.496) (end 130.302 31.496) (width 0.781439) (layer F.Cu) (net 7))
 (segment (start 130.274 31.242) (end 130.528 31.496) (width 0.781439) (layer F.Cu) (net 7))
 (segment (start 41.656 92.456) (end 45.72 92.456) (width 0.25) (layer F.Cu) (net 8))
 (segment (start 45.72 92.456) (end 48.514 89.662) (width 0.25) (layer F.Cu) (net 8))
 (segment (start 46.99 97.79) (end 47.244 98.044) (width 0.25) (layer F.Cu) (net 8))
 (segment (start 47.244 98.044) (end 47.244 90.932) (width 0.25) (layer F.Cu) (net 8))
 (segment (start 47.244 90.932) (end 48.514 89.662) (width 0.25) (layer F.Cu) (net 8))
 (segment (start 57.912 83.312) (end 62.23 83.312) (width 0.25) (layer F.Cu) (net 9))
 (segment (start 62.23 83.312) (end 62.992 82.55) (width 0.25) (layer F.Cu) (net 9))
 (segment (start 62.992 89.408) (end 62.992 95.758) (width 0.25) (layer F.Cu) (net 10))
 (segment (start 56.642 82.042) (end 56.642 85.09) (width 0.25) (layer F.Cu) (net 10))
 (segment (start 60.96 89.408) (end 62.992 89.408) (width 0.25) (layer F.Cu) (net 10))
 (segment (start 56.642 85.09) (end 60.96 89.408) (width 0.25) (layer F.Cu) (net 10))
 (segment (start 65.532 34.036) (end 67.818 34.036) (width 0.781439) (layer B.Cu) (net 11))
 (segment (start 72.644 29.21) (end 95.758 29.21) (width 0.781439) (layer B.Cu) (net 11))
 (segment (start 67.818 34.036) (end 72.644 29.21) (width 0.781439) (layer B.Cu) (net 11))
 (segment (start 65.532 39.116) (end 69.088 39.116) (width 0.781439) (layer B.Cu) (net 12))
 (segment (start 93.472 42.672) (end 95.758 44.958) (width 0.781439) (layer B.Cu) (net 12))
 (segment (start 72.644 42.672) (end 93.472 42.672) (width 0.781439) (layer B.Cu) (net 12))
 (segment (start 69.088 39.116) (end 72.644 42.672) (width 0.781439) (layer B.Cu) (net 12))
 (segment (start 41.656 94.996) (end 42.164 94.996) (width 0.25) (layer F.Cu) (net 17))
 (segment (start 42.164 94.996) (end 44.958 97.79) (width 0.25) (layer F.Cu) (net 17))
 (segment (start 44.958 97.79) (end 44.958 100.33) (width 0.25) (layer F.Cu) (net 17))
 (segment (start 44.958 100.33) (end 49.022 104.394) (width 0.25) (layer F.Cu) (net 17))
 (segment (start 49.022 104.394) (end 56.642 104.394) (width 0.25) (layer F.Cu) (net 17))
 (segment (start 56.642 104.394) (end 60.96 104.394) (width 0.25) (layer F.Cu) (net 17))
 (segment (start 60.96 104.394) (end 62.992 102.362) (width 0.25) (layer F.Cu) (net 17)))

